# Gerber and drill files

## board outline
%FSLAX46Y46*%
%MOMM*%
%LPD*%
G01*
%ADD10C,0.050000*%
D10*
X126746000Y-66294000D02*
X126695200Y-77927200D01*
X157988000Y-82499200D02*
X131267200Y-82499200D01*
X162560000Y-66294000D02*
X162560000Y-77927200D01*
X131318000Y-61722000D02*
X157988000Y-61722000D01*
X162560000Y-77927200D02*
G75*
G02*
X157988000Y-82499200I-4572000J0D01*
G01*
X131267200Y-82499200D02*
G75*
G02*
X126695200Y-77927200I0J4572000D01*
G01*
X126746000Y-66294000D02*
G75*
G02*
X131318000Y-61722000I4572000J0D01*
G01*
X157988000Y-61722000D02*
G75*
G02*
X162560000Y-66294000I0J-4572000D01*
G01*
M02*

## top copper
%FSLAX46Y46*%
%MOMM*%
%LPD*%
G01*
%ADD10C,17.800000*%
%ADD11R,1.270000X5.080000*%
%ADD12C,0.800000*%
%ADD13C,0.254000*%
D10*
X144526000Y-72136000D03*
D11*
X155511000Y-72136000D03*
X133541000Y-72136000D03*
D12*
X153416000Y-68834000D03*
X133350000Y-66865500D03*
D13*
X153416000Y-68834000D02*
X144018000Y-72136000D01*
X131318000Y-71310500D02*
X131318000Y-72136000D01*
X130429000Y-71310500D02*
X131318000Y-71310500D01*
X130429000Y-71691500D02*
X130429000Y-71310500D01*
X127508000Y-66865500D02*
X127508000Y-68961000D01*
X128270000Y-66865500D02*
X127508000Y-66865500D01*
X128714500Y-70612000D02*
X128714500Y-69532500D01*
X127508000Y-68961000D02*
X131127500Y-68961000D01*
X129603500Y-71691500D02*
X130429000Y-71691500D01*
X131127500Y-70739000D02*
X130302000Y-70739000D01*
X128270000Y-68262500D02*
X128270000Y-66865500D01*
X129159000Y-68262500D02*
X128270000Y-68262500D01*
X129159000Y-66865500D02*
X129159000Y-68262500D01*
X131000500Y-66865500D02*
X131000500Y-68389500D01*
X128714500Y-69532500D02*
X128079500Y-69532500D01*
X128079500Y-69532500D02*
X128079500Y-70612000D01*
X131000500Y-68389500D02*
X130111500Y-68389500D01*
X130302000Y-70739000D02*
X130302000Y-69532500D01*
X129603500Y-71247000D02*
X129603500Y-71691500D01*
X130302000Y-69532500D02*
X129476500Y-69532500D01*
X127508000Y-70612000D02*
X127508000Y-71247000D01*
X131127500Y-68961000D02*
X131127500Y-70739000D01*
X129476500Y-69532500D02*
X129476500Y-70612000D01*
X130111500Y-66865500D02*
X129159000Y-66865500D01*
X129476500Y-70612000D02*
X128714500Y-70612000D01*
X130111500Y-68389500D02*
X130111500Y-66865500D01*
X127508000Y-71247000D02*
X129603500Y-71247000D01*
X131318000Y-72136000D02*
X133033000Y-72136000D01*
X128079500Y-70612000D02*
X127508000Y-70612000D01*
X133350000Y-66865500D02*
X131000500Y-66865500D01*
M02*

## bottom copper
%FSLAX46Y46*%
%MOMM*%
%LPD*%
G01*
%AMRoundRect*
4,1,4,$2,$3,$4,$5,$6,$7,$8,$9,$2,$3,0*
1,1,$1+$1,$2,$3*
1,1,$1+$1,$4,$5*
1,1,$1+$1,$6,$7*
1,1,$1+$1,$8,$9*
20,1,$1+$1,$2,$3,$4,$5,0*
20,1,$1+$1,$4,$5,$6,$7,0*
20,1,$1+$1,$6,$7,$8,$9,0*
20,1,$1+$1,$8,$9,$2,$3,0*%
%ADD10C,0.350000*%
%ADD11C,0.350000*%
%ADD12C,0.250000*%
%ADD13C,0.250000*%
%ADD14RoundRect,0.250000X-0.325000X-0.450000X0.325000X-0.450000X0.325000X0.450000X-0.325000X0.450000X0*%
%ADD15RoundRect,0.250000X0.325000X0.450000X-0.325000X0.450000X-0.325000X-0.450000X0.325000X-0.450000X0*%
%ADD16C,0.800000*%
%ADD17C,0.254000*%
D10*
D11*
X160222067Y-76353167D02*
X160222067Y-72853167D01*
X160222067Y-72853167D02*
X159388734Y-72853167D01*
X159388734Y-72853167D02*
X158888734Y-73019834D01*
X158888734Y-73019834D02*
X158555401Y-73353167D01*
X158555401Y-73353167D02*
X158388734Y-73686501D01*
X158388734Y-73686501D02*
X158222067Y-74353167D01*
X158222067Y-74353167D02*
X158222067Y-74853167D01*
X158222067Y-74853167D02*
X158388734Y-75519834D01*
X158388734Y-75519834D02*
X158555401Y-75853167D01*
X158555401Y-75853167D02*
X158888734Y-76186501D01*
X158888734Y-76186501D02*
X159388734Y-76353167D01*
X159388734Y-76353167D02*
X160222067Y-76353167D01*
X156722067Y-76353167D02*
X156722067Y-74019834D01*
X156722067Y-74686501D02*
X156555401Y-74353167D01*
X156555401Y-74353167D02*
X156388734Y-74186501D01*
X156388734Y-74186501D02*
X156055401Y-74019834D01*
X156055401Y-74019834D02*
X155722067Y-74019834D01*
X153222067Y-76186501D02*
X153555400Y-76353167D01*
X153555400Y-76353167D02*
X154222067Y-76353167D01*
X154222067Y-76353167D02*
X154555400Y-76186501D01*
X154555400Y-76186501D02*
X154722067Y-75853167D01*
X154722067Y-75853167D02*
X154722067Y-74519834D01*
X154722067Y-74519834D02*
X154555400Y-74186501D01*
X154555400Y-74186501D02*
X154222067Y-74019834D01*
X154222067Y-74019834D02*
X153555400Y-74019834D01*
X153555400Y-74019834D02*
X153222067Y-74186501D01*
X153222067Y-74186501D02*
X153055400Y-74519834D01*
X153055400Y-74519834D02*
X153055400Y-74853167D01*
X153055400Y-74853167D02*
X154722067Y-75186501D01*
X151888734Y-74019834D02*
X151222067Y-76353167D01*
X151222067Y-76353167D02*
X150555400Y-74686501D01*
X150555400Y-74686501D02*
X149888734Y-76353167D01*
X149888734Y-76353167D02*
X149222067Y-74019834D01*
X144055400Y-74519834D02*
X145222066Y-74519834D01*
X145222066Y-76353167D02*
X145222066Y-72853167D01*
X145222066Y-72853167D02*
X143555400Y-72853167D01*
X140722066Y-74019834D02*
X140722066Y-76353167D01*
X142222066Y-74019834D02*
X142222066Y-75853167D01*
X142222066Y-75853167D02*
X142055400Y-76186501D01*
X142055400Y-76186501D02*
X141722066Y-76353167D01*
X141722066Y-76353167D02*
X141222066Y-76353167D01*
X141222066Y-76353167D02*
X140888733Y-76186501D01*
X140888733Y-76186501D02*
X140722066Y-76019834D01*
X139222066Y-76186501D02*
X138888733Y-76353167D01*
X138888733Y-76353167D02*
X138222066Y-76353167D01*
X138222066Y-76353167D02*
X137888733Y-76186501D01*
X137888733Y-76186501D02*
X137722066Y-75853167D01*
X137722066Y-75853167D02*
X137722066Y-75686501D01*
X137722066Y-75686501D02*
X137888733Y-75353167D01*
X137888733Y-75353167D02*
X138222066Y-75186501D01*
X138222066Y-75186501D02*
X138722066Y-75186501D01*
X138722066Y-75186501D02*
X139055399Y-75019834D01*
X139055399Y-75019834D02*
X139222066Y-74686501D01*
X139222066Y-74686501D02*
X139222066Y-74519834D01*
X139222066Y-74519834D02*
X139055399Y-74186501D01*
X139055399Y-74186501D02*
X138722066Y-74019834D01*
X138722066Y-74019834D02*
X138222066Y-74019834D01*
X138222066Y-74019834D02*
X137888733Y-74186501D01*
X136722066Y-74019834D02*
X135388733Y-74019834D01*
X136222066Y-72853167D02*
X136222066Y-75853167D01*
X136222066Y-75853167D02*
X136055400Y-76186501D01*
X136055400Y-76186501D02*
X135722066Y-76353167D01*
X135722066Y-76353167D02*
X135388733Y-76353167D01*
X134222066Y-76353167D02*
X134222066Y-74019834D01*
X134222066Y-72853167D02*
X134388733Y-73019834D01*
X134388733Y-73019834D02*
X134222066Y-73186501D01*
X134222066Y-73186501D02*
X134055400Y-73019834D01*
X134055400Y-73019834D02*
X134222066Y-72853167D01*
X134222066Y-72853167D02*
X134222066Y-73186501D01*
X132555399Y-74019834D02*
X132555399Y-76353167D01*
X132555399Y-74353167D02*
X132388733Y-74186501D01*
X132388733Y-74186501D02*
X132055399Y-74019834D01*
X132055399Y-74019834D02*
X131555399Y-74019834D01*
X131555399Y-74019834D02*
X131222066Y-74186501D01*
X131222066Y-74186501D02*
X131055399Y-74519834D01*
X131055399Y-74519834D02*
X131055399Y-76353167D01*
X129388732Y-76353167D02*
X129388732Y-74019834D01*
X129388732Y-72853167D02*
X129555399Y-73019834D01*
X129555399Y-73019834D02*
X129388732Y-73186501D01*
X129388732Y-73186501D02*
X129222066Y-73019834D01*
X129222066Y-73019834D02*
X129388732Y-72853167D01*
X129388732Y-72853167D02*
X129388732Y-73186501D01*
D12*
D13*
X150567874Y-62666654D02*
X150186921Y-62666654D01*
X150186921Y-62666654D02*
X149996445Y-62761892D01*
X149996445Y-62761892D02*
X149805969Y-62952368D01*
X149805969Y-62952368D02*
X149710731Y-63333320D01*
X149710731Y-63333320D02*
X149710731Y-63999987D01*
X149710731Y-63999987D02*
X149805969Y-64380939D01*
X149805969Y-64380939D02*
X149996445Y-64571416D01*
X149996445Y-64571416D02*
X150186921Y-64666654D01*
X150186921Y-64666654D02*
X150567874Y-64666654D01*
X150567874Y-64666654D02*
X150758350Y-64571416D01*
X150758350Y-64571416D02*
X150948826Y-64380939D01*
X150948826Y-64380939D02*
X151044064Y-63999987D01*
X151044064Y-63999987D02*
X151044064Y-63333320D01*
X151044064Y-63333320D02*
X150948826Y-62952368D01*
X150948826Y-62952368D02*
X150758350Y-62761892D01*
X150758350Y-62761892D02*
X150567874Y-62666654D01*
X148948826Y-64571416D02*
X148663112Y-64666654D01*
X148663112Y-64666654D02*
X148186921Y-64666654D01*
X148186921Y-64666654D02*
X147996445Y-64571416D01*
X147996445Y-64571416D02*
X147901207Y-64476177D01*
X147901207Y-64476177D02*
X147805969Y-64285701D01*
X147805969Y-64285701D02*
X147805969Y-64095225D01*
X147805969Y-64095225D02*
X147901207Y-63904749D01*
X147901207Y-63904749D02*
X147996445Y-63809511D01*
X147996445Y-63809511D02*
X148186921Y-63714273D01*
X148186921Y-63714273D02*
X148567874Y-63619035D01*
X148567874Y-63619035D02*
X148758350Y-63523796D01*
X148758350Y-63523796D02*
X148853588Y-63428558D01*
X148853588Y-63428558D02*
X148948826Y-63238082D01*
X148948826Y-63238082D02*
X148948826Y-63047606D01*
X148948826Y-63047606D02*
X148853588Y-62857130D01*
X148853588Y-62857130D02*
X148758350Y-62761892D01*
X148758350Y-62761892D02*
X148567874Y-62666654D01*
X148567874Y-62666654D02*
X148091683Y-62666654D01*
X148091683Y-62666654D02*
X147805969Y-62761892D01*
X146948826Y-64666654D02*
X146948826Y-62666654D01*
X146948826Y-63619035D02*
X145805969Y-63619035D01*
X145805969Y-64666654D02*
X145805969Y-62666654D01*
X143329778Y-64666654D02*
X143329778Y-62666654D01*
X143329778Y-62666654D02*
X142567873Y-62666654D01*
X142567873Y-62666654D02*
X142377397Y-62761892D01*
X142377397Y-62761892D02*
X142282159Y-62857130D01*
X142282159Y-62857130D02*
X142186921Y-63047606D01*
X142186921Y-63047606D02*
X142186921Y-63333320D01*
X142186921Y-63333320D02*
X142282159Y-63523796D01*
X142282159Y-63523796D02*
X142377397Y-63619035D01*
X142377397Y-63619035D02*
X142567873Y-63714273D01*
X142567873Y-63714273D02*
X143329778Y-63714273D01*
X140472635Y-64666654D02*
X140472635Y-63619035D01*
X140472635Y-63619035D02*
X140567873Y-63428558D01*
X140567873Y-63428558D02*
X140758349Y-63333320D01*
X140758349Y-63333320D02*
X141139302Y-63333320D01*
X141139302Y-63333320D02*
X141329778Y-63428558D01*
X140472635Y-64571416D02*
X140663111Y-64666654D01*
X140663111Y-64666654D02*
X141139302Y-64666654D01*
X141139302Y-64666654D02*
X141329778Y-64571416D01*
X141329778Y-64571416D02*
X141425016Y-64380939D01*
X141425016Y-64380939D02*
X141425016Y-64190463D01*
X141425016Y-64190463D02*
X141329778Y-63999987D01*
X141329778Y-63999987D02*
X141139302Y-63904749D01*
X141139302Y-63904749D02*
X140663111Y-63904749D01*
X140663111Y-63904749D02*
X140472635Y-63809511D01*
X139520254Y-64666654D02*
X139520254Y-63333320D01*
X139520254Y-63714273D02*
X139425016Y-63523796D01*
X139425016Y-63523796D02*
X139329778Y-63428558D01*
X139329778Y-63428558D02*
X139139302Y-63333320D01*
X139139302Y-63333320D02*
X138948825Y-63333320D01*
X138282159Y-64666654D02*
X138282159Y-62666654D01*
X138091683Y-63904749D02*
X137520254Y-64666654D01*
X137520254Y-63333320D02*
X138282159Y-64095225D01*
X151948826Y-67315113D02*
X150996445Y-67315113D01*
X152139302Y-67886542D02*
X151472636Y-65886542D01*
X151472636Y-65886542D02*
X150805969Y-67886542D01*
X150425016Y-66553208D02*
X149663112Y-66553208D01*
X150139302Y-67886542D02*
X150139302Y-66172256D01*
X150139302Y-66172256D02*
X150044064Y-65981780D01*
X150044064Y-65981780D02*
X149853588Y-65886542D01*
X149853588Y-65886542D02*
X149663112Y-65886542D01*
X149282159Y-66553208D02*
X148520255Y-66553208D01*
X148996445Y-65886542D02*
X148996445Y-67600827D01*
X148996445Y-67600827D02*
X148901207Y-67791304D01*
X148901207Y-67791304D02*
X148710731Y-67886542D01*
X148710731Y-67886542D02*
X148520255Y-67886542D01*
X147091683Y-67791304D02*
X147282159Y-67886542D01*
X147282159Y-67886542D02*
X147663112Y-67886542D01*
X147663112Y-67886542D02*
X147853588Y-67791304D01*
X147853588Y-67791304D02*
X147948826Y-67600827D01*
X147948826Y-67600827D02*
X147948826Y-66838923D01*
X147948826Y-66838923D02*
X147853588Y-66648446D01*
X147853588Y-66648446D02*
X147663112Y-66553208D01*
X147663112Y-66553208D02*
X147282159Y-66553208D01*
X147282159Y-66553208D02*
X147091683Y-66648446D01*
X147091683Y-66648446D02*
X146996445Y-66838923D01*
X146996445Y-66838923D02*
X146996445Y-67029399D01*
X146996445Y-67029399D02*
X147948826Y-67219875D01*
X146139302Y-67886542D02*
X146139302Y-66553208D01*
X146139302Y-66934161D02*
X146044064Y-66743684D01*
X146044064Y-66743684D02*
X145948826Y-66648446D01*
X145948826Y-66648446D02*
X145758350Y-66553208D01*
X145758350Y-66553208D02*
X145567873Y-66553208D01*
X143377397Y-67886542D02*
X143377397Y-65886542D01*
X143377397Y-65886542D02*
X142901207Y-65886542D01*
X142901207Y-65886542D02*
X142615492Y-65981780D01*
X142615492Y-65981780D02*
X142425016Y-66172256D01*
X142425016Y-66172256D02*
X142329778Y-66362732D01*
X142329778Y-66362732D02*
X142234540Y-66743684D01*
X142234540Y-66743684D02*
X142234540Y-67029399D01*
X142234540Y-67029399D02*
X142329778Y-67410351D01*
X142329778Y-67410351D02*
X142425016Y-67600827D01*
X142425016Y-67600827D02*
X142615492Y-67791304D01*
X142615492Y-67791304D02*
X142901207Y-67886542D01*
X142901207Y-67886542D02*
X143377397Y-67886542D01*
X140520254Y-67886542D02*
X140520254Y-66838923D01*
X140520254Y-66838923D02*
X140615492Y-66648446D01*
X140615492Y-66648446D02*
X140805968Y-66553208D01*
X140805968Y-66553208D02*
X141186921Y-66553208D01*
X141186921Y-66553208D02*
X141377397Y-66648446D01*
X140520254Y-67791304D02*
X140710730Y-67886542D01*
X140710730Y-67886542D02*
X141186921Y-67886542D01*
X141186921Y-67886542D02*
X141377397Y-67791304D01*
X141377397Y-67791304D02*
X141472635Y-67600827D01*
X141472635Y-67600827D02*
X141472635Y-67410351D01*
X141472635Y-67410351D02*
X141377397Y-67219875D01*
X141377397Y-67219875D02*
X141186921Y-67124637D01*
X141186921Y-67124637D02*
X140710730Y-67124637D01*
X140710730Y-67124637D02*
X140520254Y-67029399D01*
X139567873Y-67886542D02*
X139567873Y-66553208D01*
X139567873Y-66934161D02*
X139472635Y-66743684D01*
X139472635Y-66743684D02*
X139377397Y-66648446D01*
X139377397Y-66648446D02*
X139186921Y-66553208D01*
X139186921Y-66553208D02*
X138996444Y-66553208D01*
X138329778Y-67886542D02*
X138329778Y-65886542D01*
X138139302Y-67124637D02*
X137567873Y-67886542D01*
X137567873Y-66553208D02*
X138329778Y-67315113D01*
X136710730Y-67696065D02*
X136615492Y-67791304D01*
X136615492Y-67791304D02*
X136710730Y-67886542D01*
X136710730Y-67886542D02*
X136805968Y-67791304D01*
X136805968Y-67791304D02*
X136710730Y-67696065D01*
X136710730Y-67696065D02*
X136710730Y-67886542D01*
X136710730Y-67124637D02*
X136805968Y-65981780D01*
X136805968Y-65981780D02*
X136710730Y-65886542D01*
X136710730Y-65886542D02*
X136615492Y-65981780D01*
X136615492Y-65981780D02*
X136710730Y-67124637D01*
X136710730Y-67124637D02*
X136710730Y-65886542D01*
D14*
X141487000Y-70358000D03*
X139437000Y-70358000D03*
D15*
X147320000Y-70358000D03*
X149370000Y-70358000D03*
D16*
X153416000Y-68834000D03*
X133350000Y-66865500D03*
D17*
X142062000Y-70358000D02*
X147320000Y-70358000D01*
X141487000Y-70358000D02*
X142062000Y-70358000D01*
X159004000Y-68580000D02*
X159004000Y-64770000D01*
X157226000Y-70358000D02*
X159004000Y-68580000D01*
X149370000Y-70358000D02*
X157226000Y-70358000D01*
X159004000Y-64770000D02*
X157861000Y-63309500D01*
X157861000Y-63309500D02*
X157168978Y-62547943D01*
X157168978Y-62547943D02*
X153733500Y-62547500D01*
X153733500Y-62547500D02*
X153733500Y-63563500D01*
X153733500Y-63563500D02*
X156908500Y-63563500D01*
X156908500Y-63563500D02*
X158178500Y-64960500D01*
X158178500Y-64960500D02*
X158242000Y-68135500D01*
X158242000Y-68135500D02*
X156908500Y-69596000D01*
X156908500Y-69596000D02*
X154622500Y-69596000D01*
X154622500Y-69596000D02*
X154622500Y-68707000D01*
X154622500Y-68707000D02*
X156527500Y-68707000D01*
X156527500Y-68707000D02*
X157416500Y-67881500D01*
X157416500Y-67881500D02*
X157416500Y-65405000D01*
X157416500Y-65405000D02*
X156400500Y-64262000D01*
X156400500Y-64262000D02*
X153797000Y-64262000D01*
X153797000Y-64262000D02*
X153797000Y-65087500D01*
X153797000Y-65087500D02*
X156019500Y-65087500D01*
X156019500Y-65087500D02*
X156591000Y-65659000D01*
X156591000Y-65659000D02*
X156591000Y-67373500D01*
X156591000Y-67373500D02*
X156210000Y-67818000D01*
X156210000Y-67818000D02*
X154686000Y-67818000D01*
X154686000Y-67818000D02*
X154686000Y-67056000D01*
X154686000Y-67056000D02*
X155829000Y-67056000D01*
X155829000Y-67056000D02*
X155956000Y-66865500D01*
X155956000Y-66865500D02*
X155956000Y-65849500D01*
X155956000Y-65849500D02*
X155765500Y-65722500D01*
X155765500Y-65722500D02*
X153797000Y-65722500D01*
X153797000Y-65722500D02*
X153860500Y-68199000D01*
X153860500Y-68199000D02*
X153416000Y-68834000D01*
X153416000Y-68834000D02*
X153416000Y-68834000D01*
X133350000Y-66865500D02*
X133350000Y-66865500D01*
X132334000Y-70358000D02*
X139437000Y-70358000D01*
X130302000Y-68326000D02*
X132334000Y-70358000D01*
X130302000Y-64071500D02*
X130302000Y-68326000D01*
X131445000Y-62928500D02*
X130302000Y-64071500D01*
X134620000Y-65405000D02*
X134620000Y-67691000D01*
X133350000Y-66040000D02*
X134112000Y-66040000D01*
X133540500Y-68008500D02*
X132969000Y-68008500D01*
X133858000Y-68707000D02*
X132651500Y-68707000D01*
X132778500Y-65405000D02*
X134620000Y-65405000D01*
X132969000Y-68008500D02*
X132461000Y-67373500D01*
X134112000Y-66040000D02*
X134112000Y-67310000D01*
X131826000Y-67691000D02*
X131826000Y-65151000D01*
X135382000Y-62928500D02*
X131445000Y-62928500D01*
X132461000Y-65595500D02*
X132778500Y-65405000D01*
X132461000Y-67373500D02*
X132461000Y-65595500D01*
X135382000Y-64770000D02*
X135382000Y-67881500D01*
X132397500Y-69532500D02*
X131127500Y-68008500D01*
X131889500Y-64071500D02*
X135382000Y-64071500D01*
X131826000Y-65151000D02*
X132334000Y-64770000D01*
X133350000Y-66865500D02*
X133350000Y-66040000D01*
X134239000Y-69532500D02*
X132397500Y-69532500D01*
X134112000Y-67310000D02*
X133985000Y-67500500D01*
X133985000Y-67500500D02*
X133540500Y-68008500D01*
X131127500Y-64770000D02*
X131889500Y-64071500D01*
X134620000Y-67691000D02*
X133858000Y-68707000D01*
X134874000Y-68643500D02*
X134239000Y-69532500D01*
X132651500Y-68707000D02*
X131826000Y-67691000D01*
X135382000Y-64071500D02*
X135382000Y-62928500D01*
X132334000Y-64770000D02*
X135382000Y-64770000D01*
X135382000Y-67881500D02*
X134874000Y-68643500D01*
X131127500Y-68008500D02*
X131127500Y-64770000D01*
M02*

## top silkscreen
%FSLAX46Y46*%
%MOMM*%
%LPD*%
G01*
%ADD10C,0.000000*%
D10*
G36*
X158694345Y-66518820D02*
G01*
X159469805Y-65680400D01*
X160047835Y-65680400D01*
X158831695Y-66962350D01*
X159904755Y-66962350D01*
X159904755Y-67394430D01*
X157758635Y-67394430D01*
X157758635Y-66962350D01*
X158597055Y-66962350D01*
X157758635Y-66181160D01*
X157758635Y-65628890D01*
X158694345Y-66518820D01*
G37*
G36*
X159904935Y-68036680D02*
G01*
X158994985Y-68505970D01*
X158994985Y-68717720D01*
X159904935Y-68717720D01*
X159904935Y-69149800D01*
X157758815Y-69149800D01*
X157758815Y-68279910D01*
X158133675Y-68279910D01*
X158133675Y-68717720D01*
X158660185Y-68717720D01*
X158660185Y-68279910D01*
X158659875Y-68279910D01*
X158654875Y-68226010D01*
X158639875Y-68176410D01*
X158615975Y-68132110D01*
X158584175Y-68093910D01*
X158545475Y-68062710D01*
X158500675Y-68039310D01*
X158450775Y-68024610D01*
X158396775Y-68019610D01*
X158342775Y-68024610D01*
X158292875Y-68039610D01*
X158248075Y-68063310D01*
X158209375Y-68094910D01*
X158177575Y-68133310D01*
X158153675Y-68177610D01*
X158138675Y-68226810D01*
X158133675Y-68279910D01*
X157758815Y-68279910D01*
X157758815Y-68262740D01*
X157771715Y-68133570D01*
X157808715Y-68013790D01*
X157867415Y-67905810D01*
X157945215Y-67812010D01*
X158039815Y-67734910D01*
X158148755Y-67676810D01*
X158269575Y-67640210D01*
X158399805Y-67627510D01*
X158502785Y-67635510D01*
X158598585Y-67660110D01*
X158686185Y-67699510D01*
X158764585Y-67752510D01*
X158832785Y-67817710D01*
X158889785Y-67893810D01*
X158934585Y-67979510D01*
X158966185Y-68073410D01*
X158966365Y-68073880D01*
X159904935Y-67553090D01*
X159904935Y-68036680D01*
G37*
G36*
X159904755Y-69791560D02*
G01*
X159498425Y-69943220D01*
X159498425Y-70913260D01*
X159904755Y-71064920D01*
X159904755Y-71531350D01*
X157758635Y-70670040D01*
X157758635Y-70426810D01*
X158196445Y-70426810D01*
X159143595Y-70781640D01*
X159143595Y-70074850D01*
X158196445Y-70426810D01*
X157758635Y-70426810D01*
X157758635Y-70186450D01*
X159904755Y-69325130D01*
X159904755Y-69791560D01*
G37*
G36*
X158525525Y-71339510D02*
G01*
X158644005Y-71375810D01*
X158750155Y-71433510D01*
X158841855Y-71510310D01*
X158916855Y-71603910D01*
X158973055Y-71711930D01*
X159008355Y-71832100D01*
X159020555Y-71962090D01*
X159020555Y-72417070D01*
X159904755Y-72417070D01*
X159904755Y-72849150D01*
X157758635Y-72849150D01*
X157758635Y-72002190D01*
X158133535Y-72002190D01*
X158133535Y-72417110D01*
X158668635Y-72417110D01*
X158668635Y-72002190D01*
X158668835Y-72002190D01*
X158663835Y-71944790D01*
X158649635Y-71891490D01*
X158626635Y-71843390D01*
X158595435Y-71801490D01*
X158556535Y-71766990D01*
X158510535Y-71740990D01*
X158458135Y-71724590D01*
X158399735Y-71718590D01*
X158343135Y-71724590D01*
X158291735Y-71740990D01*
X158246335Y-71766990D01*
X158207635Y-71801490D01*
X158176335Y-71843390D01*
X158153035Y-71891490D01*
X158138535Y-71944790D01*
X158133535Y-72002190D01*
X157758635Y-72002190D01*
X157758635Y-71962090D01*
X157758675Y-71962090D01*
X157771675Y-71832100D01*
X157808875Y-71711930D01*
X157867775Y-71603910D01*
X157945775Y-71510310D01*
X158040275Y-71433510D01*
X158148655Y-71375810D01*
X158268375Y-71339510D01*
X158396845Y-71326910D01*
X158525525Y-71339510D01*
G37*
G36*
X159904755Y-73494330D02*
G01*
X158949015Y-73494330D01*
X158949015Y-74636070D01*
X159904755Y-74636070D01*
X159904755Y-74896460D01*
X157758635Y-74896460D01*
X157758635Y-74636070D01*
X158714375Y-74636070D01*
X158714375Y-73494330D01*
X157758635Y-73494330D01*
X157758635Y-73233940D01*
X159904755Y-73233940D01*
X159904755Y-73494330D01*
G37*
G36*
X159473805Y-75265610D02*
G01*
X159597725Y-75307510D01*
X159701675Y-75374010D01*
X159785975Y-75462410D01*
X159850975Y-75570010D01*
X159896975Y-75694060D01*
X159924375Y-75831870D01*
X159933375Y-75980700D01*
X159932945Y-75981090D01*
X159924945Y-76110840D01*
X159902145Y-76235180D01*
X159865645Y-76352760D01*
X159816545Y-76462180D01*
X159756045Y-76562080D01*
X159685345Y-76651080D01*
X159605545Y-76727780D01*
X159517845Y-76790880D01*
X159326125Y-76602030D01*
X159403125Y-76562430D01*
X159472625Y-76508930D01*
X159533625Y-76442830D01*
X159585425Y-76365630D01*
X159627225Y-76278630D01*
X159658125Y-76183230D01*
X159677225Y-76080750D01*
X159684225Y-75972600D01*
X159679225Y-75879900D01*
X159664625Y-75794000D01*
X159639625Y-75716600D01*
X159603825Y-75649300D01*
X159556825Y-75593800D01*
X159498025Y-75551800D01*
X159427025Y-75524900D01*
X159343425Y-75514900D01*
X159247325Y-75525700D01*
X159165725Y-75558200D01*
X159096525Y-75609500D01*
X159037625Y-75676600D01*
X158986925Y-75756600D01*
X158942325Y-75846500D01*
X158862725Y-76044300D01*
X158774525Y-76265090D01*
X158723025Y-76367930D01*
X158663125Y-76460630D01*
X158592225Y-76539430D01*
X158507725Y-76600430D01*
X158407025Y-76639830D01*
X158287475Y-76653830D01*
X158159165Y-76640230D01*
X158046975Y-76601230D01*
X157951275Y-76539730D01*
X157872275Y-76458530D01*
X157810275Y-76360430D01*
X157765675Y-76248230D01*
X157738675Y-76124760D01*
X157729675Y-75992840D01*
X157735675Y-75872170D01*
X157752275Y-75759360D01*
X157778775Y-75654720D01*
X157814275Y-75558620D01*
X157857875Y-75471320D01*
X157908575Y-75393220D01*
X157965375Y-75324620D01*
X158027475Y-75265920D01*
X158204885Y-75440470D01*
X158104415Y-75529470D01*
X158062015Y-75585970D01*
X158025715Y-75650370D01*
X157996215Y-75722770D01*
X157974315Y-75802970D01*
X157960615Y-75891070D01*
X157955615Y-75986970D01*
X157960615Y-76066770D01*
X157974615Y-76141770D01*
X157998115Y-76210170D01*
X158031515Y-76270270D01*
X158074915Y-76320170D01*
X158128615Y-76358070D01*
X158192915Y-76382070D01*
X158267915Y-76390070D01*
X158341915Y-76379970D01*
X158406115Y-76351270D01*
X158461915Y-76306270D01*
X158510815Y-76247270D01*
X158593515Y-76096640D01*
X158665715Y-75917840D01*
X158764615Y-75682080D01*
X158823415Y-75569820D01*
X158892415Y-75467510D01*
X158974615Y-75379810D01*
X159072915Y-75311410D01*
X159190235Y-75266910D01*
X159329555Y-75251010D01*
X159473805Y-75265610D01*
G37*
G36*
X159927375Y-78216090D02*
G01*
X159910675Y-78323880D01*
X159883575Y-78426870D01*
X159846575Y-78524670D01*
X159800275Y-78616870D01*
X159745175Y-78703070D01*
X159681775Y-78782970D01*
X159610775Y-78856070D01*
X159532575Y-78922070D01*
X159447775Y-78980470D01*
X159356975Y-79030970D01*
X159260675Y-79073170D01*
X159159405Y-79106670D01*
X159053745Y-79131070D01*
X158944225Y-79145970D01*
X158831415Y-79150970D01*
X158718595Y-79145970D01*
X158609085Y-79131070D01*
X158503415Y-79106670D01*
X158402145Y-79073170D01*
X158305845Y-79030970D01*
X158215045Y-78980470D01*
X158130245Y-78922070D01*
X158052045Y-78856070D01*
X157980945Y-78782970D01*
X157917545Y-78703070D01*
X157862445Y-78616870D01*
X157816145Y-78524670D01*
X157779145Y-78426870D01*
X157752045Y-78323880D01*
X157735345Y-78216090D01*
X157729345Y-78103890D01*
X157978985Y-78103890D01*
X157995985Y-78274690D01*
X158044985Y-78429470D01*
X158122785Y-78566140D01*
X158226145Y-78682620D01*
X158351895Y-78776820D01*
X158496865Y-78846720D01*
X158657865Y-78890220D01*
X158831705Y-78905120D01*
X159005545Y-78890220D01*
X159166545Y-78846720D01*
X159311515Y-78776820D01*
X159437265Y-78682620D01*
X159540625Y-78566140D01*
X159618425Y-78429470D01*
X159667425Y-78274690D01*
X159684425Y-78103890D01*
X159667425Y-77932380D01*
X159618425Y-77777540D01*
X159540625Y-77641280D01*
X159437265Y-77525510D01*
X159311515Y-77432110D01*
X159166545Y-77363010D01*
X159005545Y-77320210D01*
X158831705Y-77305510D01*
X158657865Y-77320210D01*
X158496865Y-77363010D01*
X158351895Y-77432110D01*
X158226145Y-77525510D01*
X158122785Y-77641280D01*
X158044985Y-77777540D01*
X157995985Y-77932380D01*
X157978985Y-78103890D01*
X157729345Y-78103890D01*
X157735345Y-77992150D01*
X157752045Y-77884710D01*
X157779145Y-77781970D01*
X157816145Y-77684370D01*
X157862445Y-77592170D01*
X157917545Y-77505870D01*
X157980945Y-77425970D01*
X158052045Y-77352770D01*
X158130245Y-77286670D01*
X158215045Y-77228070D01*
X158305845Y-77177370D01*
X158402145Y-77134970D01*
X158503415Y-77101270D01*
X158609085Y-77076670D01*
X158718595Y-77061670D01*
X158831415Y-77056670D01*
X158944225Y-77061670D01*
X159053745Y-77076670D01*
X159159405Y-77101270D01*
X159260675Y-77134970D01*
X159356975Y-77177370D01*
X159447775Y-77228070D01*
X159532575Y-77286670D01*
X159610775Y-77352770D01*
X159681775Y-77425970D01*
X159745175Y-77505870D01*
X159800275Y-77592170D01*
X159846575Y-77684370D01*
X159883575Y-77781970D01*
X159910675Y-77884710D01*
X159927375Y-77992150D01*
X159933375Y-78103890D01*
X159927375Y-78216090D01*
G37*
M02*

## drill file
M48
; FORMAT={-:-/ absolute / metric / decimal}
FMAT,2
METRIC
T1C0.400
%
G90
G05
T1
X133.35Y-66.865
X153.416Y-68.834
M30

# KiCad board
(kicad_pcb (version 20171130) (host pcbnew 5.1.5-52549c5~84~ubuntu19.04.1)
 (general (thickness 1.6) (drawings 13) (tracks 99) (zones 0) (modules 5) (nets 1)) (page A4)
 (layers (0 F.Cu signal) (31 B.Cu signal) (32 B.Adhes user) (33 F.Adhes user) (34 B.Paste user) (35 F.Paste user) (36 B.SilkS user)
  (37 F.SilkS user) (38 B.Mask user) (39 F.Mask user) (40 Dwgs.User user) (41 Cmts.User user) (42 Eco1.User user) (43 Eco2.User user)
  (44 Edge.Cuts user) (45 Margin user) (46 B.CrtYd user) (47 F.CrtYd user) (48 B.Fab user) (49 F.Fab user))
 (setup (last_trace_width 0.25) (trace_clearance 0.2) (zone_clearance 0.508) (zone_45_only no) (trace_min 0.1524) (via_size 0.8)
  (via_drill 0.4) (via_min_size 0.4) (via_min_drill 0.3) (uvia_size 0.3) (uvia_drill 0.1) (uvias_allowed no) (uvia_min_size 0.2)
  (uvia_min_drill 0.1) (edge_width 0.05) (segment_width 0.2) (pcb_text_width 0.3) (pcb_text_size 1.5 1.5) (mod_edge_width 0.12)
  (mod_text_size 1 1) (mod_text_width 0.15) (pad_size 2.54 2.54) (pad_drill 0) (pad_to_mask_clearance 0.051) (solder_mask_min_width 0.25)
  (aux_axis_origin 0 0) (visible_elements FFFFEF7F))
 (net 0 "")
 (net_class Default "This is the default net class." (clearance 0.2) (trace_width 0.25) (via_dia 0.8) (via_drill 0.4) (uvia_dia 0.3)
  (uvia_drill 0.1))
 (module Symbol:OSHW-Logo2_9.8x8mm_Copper (layer F.Cu) (at 131.572 79.502)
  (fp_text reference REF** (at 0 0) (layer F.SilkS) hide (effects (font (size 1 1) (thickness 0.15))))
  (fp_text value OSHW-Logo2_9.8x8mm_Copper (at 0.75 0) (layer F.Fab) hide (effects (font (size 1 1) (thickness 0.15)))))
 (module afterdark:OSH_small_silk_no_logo (layer F.Cu) (at 151.638 72.39 90)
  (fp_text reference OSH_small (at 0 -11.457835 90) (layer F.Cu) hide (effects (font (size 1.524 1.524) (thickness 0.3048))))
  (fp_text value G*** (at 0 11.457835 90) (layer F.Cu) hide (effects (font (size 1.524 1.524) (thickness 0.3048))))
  (fp_poly
   (pts (xy 6.76111 6.120635) (xy 6.20884 6.120635) (xy 5.42765 6.959055) (xy 5.42765 6.120635) (xy 4.99557 6.120635) (xy 4.99557 8.266755)
    (xy 5.42765 8.266755) (xy 5.42765 7.193695) (xy 6.7096 8.409835) (xy 6.7096 7.831805) (xy 5.87118 7.056345) (xy 6.76111 6.120635))
   (layer F.SilkS) (width 0))
  (fp_poly
   (pts (xy 4.31659 7.328185) (xy 4.11009 7.022185) (xy 3.67228 7.022185) (xy 3.67228 6.495675) (xy 4.11009 6.495675) (xy 4.16319 6.500675)
    (xy 4.21239 6.515675) (xy 4.25669 6.539575) (xy 4.29509 6.571375) (xy 4.32669 6.610075) (xy 4.35039 6.654875) (xy 4.36539 6.704775)
    (xy 4.37039 6.758775) (xy 4.36539 6.812775) (xy 4.35069 6.862675) (xy 4.32729 6.907475) (xy 4.29609 6.946175) (xy 4.25789 6.977975)
    (xy 4.21359 7.001875) (xy 4.16399 7.016875) (xy 4.11009 7.021875) (xy 4.11009 7.022185) (xy 4.31659 7.328185) (xy 4.41049 7.296585)
    (xy 4.49619 7.251785) (xy 4.57229 7.194785) (xy 4.63749 7.126585) (xy 4.69049 7.048185) (xy 4.72989 6.960585) (xy 4.75449 6.864785)
    (xy 4.76249 6.761805) (xy 4.74979 6.631575) (xy 4.71319 6.510755) (xy 4.65509 6.401815) (xy 4.57799 6.307215) (xy 4.48419 6.229415)
    (xy 4.37621 6.170715) (xy 4.25643 6.133715) (xy 4.12726 6.120815) (xy 3.2402 6.120815) (xy 3.2402 8.266935) (xy 3.67228 8.266935)
    (xy 3.67228 7.356985) (xy 3.88403 7.356985) (xy 4.35332 8.266935) (xy 4.83691 8.266935) (xy 4.31612 7.328365) (xy 4.31659 7.328185))
   (layer F.SilkS) (width 0))
  (fp_poly
   (pts (xy 2.59844 8.266755) (xy 1.96319 6.558445) (xy 2.31515 7.505595) (xy 1.60836 7.505595) (xy 1.96319 6.558445) (xy 2.59844 8.266755)
    (xy 3.06487 8.266755) (xy 2.20355 6.120635) (xy 1.71996 6.120635) (xy 0.85865 8.266755) (xy 1.32508 8.266755) (xy 1.47674 7.860425)
    (xy 2.44678 7.860425) (xy 2.59844 8.266755))
   (layer F.SilkS) (width 0))
  (fp_poly
   (pts (xy 0.42791 6.120635) (xy -0.02711 6.495535) (xy 0.38781 6.495535) (xy 0.44521 6.500535) (xy 0.49851 6.515035) (xy 0.54661 6.538335)
    (xy 0.58851 6.569635) (xy 0.62301 6.608335) (xy 0.64901 6.653735) (xy 0.66541 6.705135) (xy 0.67141 6.761735) (xy 0.66541 6.820135)
    (xy 0.64901 6.872535) (xy 0.62301 6.918535) (xy 0.58851 6.957435) (xy 0.54661 6.988635) (xy 0.49851 7.011635) (xy 0.44521 7.025835)
    (xy 0.38781 7.030835) (xy 0.38781 7.030635) (xy -0.02711 7.030635) (xy -0.02711 6.495535) (xy 0.42791 6.120635) (xy -0.45915 6.120635)
    (xy -0.45915 8.266755) (xy -0.02707 8.266755) (xy -0.02707 7.382555) (xy 0.42791 7.382555) (xy 0.5579 7.370355) (xy 0.67807 7.335055)
    (xy 0.78609 7.278855) (xy 0.87969 7.203855) (xy 0.95649 7.112155) (xy 1.01419 7.006005) (xy 1.05049 6.887525) (xy 1.06309 6.758845)
    (xy 1.05049 6.630375) (xy 1.01419 6.510655) (xy 0.95649 6.402275) (xy 0.87969 6.307775) (xy 0.78609 6.229775) (xy 0.67807 6.170875)
    (xy 0.5579 6.133675) (xy 0.42791 6.120675) (xy 0.42791 6.120635))
   (layer F.SilkS) (width 0))
  (fp_poly
   (pts (xy -1.10433 6.120635) (xy -1.10433 7.076375) (xy -2.24607 7.076375) (xy -2.24607 6.120635) (xy -2.50646 6.120635)
    (xy -2.50646 8.266755) (xy -2.24607 8.266755) (xy -2.24607 7.311015) (xy -1.10433 7.311015) (xy -1.10433 8.266755)
    (xy -0.84394 8.266755) (xy -0.84394 6.120635) (xy -1.10433 6.120635))
   (layer F.SilkS) (width 0))
  (fp_poly
   (pts (xy -3.5907 8.295375) (xy -3.44187 8.286375) (xy -3.30406 8.258975) (xy -3.18001 8.212975) (xy -3.07241 8.147975)
    (xy -2.98401 8.063675) (xy -2.91751 7.959725) (xy -2.87561 7.835805) (xy -2.86101 7.691555) (xy -2.87691 7.552235)
    (xy -2.92141 7.434915) (xy -2.98981 7.336615) (xy -3.07751 7.254415) (xy -3.17982 7.185415) (xy -3.29208 7.126615)
    (xy -3.52784 7.027715) (xy -3.70664 6.955515) (xy -3.85727 6.872815) (xy -3.91627 6.823915) (xy -3.96127 6.768115)
    (xy -3.98997 6.703915) (xy -4.00007 6.629915) (xy -3.99207 6.554915) (xy -3.96807 6.490615) (xy -3.93017 6.436915)
    (xy -3.88027 6.393515) (xy -3.82017 6.360115) (xy -3.75177 6.336615) (xy -3.67677 6.322615) (xy -3.59697 6.317615)
    (xy -3.50107 6.322615) (xy -3.41297 6.336315) (xy -3.33277 6.358215) (xy -3.26037 6.387715) (xy -3.19597 6.424015)
    (xy -3.13947 6.466415) (xy -3.05047 6.566885) (xy -2.87592 6.389475) (xy -2.93462 6.327375) (xy -3.00322 6.270575)
    (xy -3.08132 6.219875) (xy -3.16862 6.176275) (xy -3.26472 6.140775) (xy -3.36936 6.114275) (xy -3.48217 6.097675)
    (xy -3.60284 6.091675) (xy -3.73476 6.100675) (xy -3.85823 6.127675) (xy -3.97043 6.172275) (xy -4.06853 6.234275)
    (xy -4.14973 6.313275) (xy -4.21123 6.408975) (xy -4.25023 6.521165) (xy -4.26383 6.649475) (xy -4.24983 6.769025)
    (xy -4.21043 6.869725) (xy -4.14943 6.954225) (xy -4.07063 7.025125) (xy -3.97793 7.085025) (xy -3.87509 7.136525) (xy -3.6543 7.224725)
    (xy -3.4565 7.304325) (xy -3.3666 7.348925) (xy -3.2866 7.399625) (xy -3.2195 7.458525) (xy -3.1682 7.527725) (xy -3.1357 7.609325)
    (xy -3.1249 7.705425) (xy -3.1349 7.789025) (xy -3.1618 7.860025) (xy -3.2038 7.918825) (xy -3.2593 7.965825) (xy -3.3266 8.001625)
    (xy -3.404 8.026625) (xy -3.4899 8.041225) (xy -3.5826 8.046225) (xy -3.69075 8.039225) (xy -3.79323 8.020125) (xy -3.88863 7.989225)
    (xy -3.97563 7.947425) (xy -4.05283 7.895625) (xy -4.11893 7.834625) (xy -4.17243 7.765125) (xy -4.21203 7.688125)
    (xy -4.40088 7.879845) (xy -4.33778 7.967545) (xy -4.26108 8.047345) (xy -4.17208 8.118045) (xy -4.07218 8.178545)
    (xy -3.96276 8.227645) (xy -3.84518 8.264145) (xy -3.72084 8.286945) (xy -3.59109 8.294945) (xy -3.5907 8.295375))
   (layer F.SilkS) (width 0))
  (fp_poly
   (pts (xy -5.71389 8.295375) (xy -5.71389 8.046425) (xy -5.88469 8.029425) (xy -6.03947 7.980425) (xy -6.17614 7.902625)
    (xy -6.29262 7.799265) (xy -6.38682 7.673515) (xy -6.45672 7.528545) (xy -6.50022 7.367545) (xy -6.51512 7.193705)
    (xy -6.50022 7.019865) (xy -6.45672 6.858865) (xy -6.38682 6.713895) (xy -6.29262 6.588145) (xy -6.17614 6.484785)
    (xy -6.03947 6.406985) (xy -5.88469 6.357985) (xy -5.71389 6.340985) (xy -5.54238 6.357985) (xy -5.38754 6.406985)
    (xy -5.25128 6.484785) (xy -5.13551 6.588145) (xy -5.04211 6.713895) (xy -4.97301 6.858865) (xy -4.93021 7.019865)
    (xy -4.91551 7.193705) (xy -4.93021 7.367545) (xy -4.97301 7.528545) (xy -5.04211 7.673515) (xy -5.13551 7.799265)
    (xy -5.25128 7.902625) (xy -5.38754 7.980425) (xy -5.54238 8.029425) (xy -5.71389 8.046425) (xy -5.71389 8.295375)
    (xy -5.60215 8.289375) (xy -5.49471 8.272675) (xy -5.39197 8.245575) (xy -5.29437 8.208575) (xy -5.20217 8.162275)
    (xy -5.11587 8.107175) (xy -5.03597 8.043775) (xy -4.96277 7.972775) (xy -4.89667 7.894575) (xy -4.83807 7.809775)
    (xy -4.78737 7.718975) (xy -4.74497 7.622675) (xy -4.71127 7.521405) (xy -4.68667 7.415745) (xy -4.67167 7.306225)
    (xy -4.66667 7.193415) (xy -4.67167 7.080595) (xy -4.68667 6.971085) (xy -4.71127 6.865415) (xy -4.74497 6.764145)
    (xy -4.78737 6.667845) (xy -4.83807 6.577045) (xy -4.89667 6.492245) (xy -4.96277 6.414045) (xy -5.03597 6.342945)
    (xy -5.11587 6.279545) (xy -5.20217 6.224445) (xy -5.29437 6.178145) (xy -5.39197 6.141145) (xy -5.49471 6.114045)
    (xy -5.60215 6.097345) (xy -5.71389 6.091345) (xy -5.82609 6.097345) (xy -5.93388 6.114045) (xy -6.03687 6.141145)
    (xy -6.13467 6.178145) (xy -6.22687 6.224445) (xy -6.31307 6.279545) (xy -6.39297 6.342945) (xy -6.46607 6.414045)
    (xy -6.53207 6.492245) (xy -6.59047 6.577045) (xy -6.64097 6.667845) (xy -6.68317 6.764145) (xy -6.71667 6.865415)
    (xy -6.74107 6.971085) (xy -6.75597 7.080595) (xy -6.76097 7.193415) (xy -6.75597 7.306225) (xy -6.74107 7.415745)
    (xy -6.71667 7.521405) (xy -6.68317 7.622675) (xy -6.64097 7.718975) (xy -6.59047 7.809775) (xy -6.53207 7.894575)
    (xy -6.46607 7.972775) (xy -6.39297 8.043775) (xy -6.31307 8.107175) (xy -6.22687 8.162275) (xy -6.13467 8.208575)
    (xy -6.03687 8.245575) (xy -5.93388 8.272675) (xy -5.82609 8.289375) (xy -5.71389 8.295375))
   (layer F.SilkS) (width 0)))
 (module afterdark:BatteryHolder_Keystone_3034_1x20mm (layer F.Cu) (at 144.526 72.136)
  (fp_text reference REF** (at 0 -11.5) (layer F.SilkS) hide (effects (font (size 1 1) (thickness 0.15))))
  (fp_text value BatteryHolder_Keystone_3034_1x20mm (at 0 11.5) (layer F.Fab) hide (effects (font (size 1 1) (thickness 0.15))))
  (pad 2 smd circle (at 0 0) (size 17.8 17.8) (layers F.Cu F.Mask))
  (pad 1 smd rect (at 10.985 0) (size 1.27 5.08) (layers F.Cu F.Paste F.Mask))
  (pad 1 smd rect (at -10.985 0) (size 1.27 5.08) (layers F.Cu F.Paste F.Mask)))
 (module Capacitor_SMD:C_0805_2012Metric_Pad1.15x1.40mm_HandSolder (layer B.Cu) (at 140.462 70.358)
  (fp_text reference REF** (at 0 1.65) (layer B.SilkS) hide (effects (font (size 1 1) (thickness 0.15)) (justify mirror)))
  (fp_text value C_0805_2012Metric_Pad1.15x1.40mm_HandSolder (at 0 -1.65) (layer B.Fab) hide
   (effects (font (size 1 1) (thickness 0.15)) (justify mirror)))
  (pad 2 smd roundrect (at 1.025 0) (size 1.15 1.4) (layers B.Cu B.Paste B.Mask) (roundrect_rratio 0.217391))
  (pad 1 smd roundrect (at -1.025 0) (size 1.15 1.4) (layers B.Cu B.Paste B.Mask) (roundrect_rratio 0.217391)))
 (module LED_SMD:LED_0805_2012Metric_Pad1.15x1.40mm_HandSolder (layer B.Cu) (at 148.345 70.358 180)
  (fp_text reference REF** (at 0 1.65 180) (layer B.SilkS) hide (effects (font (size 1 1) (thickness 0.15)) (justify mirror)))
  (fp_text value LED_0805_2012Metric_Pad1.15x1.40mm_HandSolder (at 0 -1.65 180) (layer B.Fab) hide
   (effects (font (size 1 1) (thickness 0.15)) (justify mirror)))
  (pad 2 smd roundrect (at 1.025 0 180) (size 1.15 1.4) (layers B.Cu B.Paste B.Mask) (roundrect_rratio 0.217391))
  (pad 1 smd roundrect (at -1.025 0 180) (size 1.15 1.4) (layers B.Cu B.Paste B.Mask) (roundrect_rratio 0.217391)))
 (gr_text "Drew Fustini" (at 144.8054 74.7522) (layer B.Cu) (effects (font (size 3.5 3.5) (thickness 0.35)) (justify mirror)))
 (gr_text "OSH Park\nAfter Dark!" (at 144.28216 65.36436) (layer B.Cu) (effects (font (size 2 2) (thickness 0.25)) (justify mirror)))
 (gr_line (start 126.746 66.294) (end 126.6952 77.9272) (layer Edge.Cuts) (width 0.05))
 (gr_line (start 157.988 82.4992) (end 131.2672 82.4992) (layer Edge.Cuts) (width 0.05))
 (gr_line (start 162.56 66.294) (end 162.56 77.9272) (layer Edge.Cuts) (width 0.05))
 (gr_line (start 131.318 61.722) (end 157.988 61.722) (layer Edge.Cuts) (width 0.05))
 (gr_arc (start 157.988 77.9272) (end 157.988 82.4992) (angle -90) (layer Edge.Cuts) (width 0.05))
 (gr_arc (start 131.2672 77.9272) (end 126.6952 77.9272) (angle -90) (layer Edge.Cuts) (width 0.05))
 (gr_arc (start 131.318 66.294) (end 131.318 61.722) (angle -90) (layer Edge.Cuts) (width 0.05))
 (gr_arc (start 157.988 66.294) (end 162.56 66.294) (angle -90) (layer Edge.Cuts) (width 0.05))
 (segment (start 142.062 70.358) (end 147.32 70.358) (width 0.254) (layer B.Cu) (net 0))
 (segment (start 141.487 70.358) (end 142.062 70.358) (width 0.254) (layer B.Cu) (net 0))
 (segment (start 159.004 68.58) (end 159.004 64.77) (width 0.254) (layer B.Cu) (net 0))
 (segment (start 157.226 70.358) (end 159.004 68.58) (width 0.254) (layer B.Cu) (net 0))
 (segment (start 149.37 70.358) (end 157.226 70.358) (width 0.254) (layer B.Cu) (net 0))
 (segment (start 159.004 64.77) (end 157.861 63.3095) (width 0.254) (layer B.Cu) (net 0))
 (segment (start 157.861 63.3095) (end 157.168978 62.547943) (width 0.254) (layer B.Cu) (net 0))
 (segment (start 157.168978 62.547943) (end 153.7335 62.5475) (width 0.254) (layer B.Cu) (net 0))
 (segment (start 153.7335 62.5475) (end 153.7335 63.5635) (width 0.254) (layer B.Cu) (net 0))
 (segment (start 153.7335 63.5635) (end 156.9085 63.5635) (width 0.254) (layer B.Cu) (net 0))
 (segment (start 156.9085 63.5635) (end 158.1785 64.9605) (width 0.254) (layer B.Cu) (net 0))
 (segment (start 158.1785 64.9605) (end 158.242 68.1355) (width 0.254) (layer B.Cu) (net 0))
 (segment (start 158.242 68.1355) (end 156.9085 69.596) (width 0.254) (layer B.Cu) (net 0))
 (segment (start 156.9085 69.596) (end 154.6225 69.596) (width 0.254) (layer B.Cu) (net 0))
 (segment (start 154.6225 69.596) (end 154.6225 68.707) (width 0.254) (layer B.Cu) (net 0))
 (segment (start 154.6225 68.707) (end 156.5275 68.707) (width 0.254) (layer B.Cu) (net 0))
 (segment (start 156.5275 68.707) (end 157.4165 67.8815) (width 0.254) (layer B.Cu) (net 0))
 (segment (start 157.4165 67.8815) (end 157.4165 65.405) (width 0.254) (layer B.Cu) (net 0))
 (segment (start 157.4165 65.405) (end 156.4005 64.262) (width 0.254) (layer B.Cu) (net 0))
 (segment (start 156.4005 64.262) (end 153.797 64.262) (width 0.254) (layer B.Cu) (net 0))
 (segment (start 153.797 64.262) (end 153.797 65.0875) (width 0.254) (layer B.Cu) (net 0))
 (segment (start 153.797 65.0875) (end 156.0195 65.0875) (width 0.254) (layer B.Cu) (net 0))
 (segment (start 156.0195 65.0875) (end 156.591 65.659) (width 0.254) (layer B.Cu) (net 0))
 (segment (start 156.591 65.659) (end 156.591 67.3735) (width 0.254) (layer B.Cu) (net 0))
 (segment (start 156.591 67.3735) (end 156.21 67.818) (width 0.254) (layer B.Cu) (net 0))
 (segment (start 156.21 67.818) (end 154.686 67.818) (width 0.254) (layer B.Cu) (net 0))
 (segment (start 154.686 67.818) (end 154.686 67.056) (width 0.254) (layer B.Cu) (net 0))
 (segment (start 154.686 67.056) (end 155.829 67.056) (width 0.254) (layer B.Cu) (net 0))
 (segment (start 155.829 67.056) (end 155.956 66.8655) (width 0.254) (layer B.Cu) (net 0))
 (segment (start 155.956 66.8655) (end 155.956 65.8495) (width 0.254) (layer B.Cu) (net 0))
 (segment (start 155.956 65.8495) (end 155.7655 65.7225) (width 0.254) (layer B.Cu) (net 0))
 (segment (start 155.7655 65.7225) (end 153.797 65.7225) (width 0.254) (layer B.Cu) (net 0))
 (segment (start 153.797 65.7225) (end 153.8605 68.199) (width 0.254) (layer B.Cu) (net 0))
 (segment (start 153.8605 68.199) (end 153.416 68.834) (width 0.254) (layer B.Cu) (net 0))
 (segment (start 153.416 68.834) (end 153.416 68.834) (width 0.254) (layer B.Cu) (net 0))
 (via (at 153.416 68.834) (size 0.8) (drill 0.4) (layers F.Cu B.Cu) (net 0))
 (segment (start 153.416 68.834) (end 144.018 72.136) (width 0.254) (layer F.Cu) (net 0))
 (segment (start 131.318 71.3105) (end 131.318 72.136) (width 0.254) (layer F.Cu) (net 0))
 (segment (start 130.429 71.3105) (end 131.318 71.3105) (width 0.254) (layer F.Cu) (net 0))
 (segment (start 130.429 71.6915) (end 130.429 71.3105) (width 0.254) (layer F.Cu) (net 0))
 (segment (start 127.508 66.8655) (end 127.508 68.961) (width 0.254) (layer F.Cu) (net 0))
 (segment (start 128.27 66.8655) (end 127.508 66.8655) (width 0.254) (layer F.Cu) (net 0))
 (segment (start 128.7145 70.612) (end 128.7145 69.5325) (width 0.254) (layer F.Cu) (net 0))
 (segment (start 127.508 68.961) (end 131.1275 68.961) (width 0.254) (layer F.Cu) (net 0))
 (segment (start 129.6035 71.6915) (end 130.429 71.6915) (width 0.254) (layer F.Cu) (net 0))
 (segment (start 131.1275 70.739) (end 130.302 70.739) (width 0.254) (layer F.Cu) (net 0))
 (segment (start 128.27 68.2625) (end 128.27 66.8655) (width 0.254) (layer F.Cu) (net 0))
 (segment (start 129.159 68.2625) (end 128.27 68.2625) (width 0.254) (layer F.Cu) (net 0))
 (segment (start 129.159 66.8655) (end 129.159 68.2625) (width 0.254) (layer F.Cu) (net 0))
 (segment (start 131.0005 66.8655) (end 131.0005 68.3895) (width 0.254) (layer F.Cu) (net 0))
 (segment (start 128.7145 69.5325) (end 128.0795 69.5325) (width 0.254) (layer F.Cu) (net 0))
 (segment (start 128.0795 69.5325) (end 128.0795 70.612) (width 0.254) (layer F.Cu) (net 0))
 (segment (start 131.0005 68.3895) (end 130.1115 68.3895) (width 0.254) (layer F.Cu) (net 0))
 (segment (start 130.302 70.739) (end 130.302 69.5325) (width 0.254) (layer F.Cu) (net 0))
 (segment (start 129.6035 71.247) (end 129.6035 71.6915) (width 0.254) (layer F.Cu) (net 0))
 (segment (start 130.302 69.5325) (end 129.4765 69.5325) (width 0.254) (layer F.Cu) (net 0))
 (segment (start 127.508 70.612) (end 127.508 71.247) (width 0.254) (layer F.Cu) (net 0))
 (segment (start 131.1275 68.961) (end 131.1275 70.739) (width 0.254) (layer F.Cu) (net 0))
 (segment (start 129.4765 69.5325) (end 129.4765 70.612) (width 0.254) (layer F.Cu) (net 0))
 (segment (start 130.1115 66.8655) (end 129.159 66.8655) (width 0.254) (layer F.Cu) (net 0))
 (segment (start 129.4765 70.612) (end 128.7145 70.612) (width 0.254) (layer F.Cu) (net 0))
 (segment (start 130.1115 68.3895) (end 130.1115 66.8655) (width 0.254) (layer F.Cu) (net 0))
 (segment (start 127.508 71.247) (end 129.6035 71.247) (width 0.254) (layer F.Cu) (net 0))
 (segment (start 131.318 72.136) (end 133.033 72.136) (width 0.254) (layer F.Cu) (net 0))
 (segment (start 128.0795 70.612) (end 127.508 70.612) (width 0.254) (layer F.Cu) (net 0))
 (segment (start 133.35 66.8655) (end 131.0005 66.8655) (width 0.254) (layer F.Cu) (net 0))
 (segment (start 133.35 66.8655) (end 133.35 66.8655) (width 0.254) (layer B.Cu) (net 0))
 (via (at 133.35 66.8655) (size 0.8) (drill 0.4) (layers F.Cu B.Cu) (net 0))
 (segment (start 132.334 70.358) (end 139.437 70.358) (width 0.254) (layer B.Cu) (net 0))
 (segment (start 130.302 68.326) (end 132.334 70.358) (width 0.254) (layer B.Cu) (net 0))
 (segment (start 130.302 64.0715) (end 130.302 68.326) (width 0.254) (layer B.Cu) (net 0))
 (segment (start 131.445 62.9285) (end 130.302 64.0715) (width 0.254) (layer B.Cu) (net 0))
 (segment (start 134.62 65.405) (end 134.62 67.691) (width 0.254) (layer B.Cu) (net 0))
 (segment (start 133.35 66.04) (end 134.112 66.04) (width 0.254) (layer B.Cu) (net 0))
 (segment (start 133.5405 68.0085) (end 132.969 68.0085) (width 0.254) (layer B.Cu) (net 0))
 (segment (start 133.858 68.707) (end 132.6515 68.707) (width 0.254) (layer B.Cu) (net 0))
 (segment (start 132.7785 65.405) (end 134.62 65.405) (width 0.254) (layer B.Cu) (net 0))
 (segment (start 132.969 68.0085) (end 132.461 67.3735) (width 0.254) (layer B.Cu) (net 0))
 (segment (start 134.112 66.04) (end 134.112 67.31) (width 0.254) (layer B.Cu) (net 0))
 (segment (start 131.826 67.691) (end 131.826 65.151) (width 0.254) (layer B.Cu) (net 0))
 (segment (start 135.382 62.9285) (end 131.445 62.9285) (width 0.254) (layer B.Cu) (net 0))
 (segment (start 132.461 65.5955) (end 132.7785 65.405) (width 0.254) (layer B.Cu) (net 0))
 (segment (start 132.461 67.3735) (end 132.461 65.5955) (width 0.254) (layer B.Cu) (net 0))
 (segment (start 135.382 64.77) (end 135.382 67.8815) (width 0.254) (layer B.Cu) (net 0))
 (segment (start 132.3975 69.5325) (end 131.1275 68.0085) (width 0.254) (layer B.Cu) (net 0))
 (segment (start 131.8895 64.0715) (end 135.382 64.0715) (width 0.254) (layer B.Cu) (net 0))
 (segment (start 131.826 65.151) (end 132.334 64.77) (width 0.254) (layer B.Cu) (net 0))
 (segment (start 133.35 66.8655) (end 133.35 66.04) (width 0.254) (layer B.Cu) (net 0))
 (segment (start 134.239 69.5325) (end 132.3975 69.5325) (width 0.254) (layer B.Cu) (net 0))
 (segment (start 134.112 67.31) (end 133.985 67.5005) (width 0.254) (layer B.Cu) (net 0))
 (segment (start 133.985 67.5005) (end 133.5405 68.0085) (width 0.254) (layer B.Cu) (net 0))
 (segment (start 131.1275 64.77) (end 131.8895 64.0715) (width 0.254) (layer B.Cu) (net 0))
 (segment (start 134.62 67.691) (end 133.858 68.707) (width 0.254) (layer B.Cu) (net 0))
 (segment (start 134.874 68.6435) (end 134.239 69.5325) (width 0.254) (layer B.Cu) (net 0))
 (segment (start 132.6515 68.707) (end 131.826 67.691) (width 0.254) (layer B.Cu) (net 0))
 (segment (start 135.382 64.0715) (end 135.382 62.9285) (width 0.254) (layer B.Cu) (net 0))
 (segment (start 132.334 64.77) (end 135.382 64.77) (width 0.254) (layer B.Cu) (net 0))
 (segment (start 135.382 67.8815) (end 134.874 68.6435) (width 0.254) (layer B.Cu) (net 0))
 (segment (start 131.1275 68.0085) (end 131.1275 64.77) (width 0.254) (layer B.Cu) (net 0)))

